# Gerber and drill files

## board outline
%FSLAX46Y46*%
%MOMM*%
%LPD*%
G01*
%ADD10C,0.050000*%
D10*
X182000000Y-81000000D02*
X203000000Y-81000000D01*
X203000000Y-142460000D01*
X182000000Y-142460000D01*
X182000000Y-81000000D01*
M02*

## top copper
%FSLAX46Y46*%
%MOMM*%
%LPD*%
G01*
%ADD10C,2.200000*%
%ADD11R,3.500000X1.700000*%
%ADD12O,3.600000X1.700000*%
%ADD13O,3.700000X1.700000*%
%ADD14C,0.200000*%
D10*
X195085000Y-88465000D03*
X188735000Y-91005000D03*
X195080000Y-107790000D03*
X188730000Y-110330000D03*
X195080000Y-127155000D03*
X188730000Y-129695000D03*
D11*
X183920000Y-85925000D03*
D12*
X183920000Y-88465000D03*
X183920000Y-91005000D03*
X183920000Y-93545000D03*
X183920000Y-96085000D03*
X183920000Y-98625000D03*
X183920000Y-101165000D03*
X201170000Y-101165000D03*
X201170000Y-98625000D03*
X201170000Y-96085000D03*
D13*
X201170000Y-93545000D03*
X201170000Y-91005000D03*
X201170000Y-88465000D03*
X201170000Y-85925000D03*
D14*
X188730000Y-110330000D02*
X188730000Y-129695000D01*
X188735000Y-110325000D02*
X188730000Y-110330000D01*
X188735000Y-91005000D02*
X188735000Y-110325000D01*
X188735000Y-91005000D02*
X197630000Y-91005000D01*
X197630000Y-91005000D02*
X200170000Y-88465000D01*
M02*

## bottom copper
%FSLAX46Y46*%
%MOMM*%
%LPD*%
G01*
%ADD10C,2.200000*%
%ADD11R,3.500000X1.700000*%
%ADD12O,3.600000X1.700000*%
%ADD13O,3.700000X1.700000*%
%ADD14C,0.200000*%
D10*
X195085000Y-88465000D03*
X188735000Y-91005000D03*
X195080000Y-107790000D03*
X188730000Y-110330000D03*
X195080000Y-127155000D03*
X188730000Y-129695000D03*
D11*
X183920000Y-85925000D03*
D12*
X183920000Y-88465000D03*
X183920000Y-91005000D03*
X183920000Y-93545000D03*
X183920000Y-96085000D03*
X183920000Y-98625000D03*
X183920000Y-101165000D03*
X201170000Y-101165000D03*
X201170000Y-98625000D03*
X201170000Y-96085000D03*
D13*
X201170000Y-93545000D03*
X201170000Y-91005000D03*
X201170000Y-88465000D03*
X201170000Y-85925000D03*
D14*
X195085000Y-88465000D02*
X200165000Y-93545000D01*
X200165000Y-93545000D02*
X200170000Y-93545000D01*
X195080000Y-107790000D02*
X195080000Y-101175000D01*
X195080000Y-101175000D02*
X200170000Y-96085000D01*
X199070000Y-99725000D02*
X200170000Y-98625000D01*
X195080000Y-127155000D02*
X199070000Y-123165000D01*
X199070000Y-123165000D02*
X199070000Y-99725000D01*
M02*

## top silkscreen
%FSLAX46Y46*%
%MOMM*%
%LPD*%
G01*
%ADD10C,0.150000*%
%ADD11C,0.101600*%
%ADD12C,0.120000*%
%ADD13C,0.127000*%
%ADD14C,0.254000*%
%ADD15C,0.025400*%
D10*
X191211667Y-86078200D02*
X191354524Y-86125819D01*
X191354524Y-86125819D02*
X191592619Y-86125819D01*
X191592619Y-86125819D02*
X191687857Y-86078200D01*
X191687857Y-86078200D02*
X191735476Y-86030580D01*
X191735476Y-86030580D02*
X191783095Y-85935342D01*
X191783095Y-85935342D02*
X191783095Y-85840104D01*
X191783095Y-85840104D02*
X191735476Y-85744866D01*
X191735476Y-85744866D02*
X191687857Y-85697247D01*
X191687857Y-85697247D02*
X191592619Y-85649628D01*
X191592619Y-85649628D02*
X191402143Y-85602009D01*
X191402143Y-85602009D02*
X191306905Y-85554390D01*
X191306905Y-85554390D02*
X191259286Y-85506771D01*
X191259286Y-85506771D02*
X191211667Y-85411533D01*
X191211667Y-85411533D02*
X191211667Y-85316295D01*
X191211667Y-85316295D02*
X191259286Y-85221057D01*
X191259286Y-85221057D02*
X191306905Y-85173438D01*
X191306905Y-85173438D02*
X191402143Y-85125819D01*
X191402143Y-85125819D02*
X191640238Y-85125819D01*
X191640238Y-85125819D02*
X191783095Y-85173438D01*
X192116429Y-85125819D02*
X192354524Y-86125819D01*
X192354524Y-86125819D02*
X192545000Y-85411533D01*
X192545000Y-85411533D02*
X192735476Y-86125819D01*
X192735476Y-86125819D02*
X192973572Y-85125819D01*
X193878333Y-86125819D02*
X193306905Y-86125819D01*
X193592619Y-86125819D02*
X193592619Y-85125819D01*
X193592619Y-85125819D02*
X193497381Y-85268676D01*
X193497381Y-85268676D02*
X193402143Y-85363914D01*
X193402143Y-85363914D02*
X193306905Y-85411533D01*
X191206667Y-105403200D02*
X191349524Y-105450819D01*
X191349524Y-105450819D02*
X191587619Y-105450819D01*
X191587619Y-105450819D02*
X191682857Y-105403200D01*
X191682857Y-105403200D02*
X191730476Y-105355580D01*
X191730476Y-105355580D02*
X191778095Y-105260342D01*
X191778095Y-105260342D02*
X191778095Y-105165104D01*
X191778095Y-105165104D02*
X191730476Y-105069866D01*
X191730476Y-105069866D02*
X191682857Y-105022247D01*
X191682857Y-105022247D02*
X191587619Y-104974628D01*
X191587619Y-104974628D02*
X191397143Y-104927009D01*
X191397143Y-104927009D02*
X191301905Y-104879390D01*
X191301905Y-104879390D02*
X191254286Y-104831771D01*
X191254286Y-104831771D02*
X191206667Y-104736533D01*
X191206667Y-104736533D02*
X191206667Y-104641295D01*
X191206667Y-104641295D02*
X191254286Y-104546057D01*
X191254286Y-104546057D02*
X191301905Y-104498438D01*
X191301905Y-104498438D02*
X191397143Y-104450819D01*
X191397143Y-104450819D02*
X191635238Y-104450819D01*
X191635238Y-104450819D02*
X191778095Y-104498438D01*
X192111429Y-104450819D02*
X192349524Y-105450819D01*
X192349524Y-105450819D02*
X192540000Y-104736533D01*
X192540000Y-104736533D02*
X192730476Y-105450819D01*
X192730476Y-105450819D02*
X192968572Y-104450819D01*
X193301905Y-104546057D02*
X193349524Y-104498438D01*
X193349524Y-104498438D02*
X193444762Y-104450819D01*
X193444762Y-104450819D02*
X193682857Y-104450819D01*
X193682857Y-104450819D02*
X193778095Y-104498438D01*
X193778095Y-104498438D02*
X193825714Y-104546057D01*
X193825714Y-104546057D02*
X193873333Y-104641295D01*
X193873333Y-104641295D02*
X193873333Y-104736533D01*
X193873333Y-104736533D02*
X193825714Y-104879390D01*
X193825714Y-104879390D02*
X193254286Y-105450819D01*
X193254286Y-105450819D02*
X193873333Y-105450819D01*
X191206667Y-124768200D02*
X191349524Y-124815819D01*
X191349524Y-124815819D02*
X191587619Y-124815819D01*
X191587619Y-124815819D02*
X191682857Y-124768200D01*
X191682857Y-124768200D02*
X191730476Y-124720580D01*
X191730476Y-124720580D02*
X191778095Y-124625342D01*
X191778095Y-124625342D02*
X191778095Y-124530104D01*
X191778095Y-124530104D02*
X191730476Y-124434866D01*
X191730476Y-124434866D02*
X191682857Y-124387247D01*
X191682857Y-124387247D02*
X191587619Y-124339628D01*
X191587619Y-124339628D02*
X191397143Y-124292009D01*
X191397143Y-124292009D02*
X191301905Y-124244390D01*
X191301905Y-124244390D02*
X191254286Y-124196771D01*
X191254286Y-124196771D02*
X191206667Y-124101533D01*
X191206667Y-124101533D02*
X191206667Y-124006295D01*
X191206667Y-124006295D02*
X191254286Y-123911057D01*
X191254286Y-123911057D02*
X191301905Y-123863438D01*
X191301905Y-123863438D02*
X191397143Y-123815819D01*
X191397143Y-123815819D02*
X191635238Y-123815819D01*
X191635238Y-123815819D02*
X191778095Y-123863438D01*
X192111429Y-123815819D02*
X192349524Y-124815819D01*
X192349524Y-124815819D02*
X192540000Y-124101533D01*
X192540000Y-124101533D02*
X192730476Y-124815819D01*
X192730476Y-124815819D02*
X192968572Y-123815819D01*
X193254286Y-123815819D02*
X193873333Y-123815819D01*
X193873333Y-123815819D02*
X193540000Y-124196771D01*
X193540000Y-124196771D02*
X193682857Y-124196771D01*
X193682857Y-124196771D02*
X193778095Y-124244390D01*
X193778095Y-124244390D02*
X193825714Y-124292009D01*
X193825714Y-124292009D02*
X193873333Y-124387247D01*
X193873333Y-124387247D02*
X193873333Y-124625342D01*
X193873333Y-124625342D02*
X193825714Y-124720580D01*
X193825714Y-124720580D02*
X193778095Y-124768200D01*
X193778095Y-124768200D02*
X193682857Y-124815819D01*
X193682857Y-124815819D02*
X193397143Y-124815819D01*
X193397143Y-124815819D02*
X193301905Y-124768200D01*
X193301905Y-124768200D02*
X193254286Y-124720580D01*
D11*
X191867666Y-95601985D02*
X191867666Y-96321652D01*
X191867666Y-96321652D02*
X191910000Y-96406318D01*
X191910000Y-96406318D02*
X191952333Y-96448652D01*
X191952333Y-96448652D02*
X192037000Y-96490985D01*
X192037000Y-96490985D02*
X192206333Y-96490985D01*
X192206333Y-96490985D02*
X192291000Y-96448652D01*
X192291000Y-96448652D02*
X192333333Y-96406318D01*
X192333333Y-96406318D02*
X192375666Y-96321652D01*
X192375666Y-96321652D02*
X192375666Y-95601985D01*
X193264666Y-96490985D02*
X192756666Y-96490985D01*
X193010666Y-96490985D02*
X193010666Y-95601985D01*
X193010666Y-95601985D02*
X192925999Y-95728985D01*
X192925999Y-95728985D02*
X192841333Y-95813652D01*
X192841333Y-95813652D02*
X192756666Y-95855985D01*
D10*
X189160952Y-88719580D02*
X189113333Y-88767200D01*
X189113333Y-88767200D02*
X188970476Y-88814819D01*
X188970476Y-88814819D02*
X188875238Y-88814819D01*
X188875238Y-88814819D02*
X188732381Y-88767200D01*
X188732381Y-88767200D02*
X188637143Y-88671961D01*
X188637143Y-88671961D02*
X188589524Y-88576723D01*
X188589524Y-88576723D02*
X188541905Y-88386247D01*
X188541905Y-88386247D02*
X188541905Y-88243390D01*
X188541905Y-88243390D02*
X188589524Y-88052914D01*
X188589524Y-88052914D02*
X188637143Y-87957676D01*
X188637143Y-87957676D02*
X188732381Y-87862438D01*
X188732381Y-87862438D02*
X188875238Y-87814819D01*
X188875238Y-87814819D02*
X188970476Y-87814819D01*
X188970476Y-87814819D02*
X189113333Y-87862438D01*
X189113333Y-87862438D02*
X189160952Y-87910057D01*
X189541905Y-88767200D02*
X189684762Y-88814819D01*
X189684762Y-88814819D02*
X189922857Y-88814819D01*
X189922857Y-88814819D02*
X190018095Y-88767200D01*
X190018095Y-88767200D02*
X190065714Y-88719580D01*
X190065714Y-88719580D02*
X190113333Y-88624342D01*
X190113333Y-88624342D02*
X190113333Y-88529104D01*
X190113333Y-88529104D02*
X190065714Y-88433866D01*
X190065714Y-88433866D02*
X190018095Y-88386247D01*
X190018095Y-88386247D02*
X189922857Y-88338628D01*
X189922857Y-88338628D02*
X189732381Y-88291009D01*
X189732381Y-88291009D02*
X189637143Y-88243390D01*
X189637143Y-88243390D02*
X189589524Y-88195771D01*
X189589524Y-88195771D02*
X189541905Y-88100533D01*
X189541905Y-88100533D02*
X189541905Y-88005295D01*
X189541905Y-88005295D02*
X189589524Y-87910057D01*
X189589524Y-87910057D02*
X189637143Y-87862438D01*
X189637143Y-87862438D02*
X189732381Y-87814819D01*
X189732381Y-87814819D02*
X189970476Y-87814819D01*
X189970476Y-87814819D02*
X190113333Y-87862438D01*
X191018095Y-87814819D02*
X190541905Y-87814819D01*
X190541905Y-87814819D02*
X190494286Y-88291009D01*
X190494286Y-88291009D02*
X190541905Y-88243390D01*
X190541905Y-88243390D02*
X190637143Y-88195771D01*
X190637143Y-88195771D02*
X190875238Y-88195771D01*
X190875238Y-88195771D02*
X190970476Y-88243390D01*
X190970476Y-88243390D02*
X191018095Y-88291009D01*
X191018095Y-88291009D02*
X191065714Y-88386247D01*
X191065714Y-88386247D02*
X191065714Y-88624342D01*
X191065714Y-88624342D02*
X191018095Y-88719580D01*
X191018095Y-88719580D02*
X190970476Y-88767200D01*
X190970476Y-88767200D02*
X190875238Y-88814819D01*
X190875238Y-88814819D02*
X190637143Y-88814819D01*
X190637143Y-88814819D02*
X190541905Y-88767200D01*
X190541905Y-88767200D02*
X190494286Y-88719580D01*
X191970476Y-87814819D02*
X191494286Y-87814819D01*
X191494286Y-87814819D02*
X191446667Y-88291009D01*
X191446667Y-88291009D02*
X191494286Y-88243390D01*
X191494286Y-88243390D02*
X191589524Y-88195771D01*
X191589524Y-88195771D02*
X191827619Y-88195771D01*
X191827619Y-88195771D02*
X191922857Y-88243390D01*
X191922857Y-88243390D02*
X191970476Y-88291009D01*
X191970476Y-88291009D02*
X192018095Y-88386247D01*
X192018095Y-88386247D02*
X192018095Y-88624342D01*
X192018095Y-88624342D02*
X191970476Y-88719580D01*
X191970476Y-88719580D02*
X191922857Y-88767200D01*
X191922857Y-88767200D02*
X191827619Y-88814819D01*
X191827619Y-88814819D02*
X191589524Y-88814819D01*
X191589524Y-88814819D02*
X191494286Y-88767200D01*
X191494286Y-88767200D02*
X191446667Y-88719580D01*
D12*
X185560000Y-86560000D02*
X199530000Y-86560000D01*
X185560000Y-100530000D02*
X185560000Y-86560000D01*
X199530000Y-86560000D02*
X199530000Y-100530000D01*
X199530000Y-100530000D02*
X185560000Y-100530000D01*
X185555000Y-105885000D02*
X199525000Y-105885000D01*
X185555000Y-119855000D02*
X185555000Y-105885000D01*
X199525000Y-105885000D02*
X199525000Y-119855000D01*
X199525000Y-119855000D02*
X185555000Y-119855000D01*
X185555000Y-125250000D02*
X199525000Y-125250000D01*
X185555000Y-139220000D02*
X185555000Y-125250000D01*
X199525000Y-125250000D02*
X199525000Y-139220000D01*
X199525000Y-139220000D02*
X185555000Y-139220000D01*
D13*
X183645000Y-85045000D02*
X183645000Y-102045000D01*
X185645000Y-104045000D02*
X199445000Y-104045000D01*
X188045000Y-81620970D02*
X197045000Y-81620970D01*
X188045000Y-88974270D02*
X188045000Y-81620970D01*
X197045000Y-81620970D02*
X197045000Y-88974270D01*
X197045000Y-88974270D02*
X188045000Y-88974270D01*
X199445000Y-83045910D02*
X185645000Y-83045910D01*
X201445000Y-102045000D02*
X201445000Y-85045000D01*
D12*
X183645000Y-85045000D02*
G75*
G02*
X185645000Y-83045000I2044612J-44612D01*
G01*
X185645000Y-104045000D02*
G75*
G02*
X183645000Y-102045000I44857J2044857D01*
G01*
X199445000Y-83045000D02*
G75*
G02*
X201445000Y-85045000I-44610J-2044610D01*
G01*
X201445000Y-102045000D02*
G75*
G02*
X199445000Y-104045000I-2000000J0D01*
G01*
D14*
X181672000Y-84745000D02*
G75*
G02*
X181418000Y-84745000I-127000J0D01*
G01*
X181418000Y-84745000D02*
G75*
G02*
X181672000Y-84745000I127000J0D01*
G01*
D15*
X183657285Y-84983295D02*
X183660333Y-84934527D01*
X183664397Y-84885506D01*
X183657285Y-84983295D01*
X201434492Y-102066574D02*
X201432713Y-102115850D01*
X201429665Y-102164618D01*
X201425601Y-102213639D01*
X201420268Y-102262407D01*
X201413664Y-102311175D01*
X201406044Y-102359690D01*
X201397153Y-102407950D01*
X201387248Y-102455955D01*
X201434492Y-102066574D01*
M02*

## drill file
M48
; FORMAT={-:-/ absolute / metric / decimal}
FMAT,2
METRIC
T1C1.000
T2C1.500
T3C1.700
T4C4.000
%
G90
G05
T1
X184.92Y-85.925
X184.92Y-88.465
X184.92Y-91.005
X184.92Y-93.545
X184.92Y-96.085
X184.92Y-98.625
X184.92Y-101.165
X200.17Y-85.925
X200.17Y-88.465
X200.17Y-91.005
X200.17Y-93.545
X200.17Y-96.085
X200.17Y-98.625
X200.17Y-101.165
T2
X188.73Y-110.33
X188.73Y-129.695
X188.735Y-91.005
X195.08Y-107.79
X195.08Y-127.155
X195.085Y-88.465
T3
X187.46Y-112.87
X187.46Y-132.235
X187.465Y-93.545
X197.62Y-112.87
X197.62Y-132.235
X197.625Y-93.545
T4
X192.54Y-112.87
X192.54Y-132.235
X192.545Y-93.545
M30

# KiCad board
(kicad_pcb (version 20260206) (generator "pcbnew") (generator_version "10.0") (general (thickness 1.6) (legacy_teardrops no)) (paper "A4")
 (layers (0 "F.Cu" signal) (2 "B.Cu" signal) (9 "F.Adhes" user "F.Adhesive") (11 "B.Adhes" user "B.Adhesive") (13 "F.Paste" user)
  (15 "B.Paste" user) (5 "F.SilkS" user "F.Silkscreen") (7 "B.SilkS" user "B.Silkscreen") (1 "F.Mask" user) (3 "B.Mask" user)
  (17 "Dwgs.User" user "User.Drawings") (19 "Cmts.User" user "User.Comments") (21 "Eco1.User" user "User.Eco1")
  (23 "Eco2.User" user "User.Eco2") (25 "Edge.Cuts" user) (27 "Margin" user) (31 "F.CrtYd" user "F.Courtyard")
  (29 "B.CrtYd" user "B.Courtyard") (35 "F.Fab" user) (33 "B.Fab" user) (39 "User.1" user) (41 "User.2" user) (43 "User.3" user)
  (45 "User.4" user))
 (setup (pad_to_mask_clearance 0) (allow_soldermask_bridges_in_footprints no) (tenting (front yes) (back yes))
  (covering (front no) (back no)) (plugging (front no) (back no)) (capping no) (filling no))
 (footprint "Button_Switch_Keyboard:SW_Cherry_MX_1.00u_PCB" (layer "F.Cu") (at 195.085 88.465)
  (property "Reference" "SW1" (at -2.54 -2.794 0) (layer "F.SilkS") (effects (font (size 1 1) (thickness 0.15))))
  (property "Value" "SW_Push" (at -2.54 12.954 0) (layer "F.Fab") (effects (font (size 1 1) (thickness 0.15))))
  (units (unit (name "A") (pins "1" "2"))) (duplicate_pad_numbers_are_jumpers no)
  (fp_line (start -9.525 -1.905) (end 4.445 -1.905) (stroke (width 0.12) (type solid)) (layer "F.SilkS"))
  (fp_line (start -9.525 12.065) (end -9.525 -1.905) (stroke (width 0.12) (type solid)) (layer "F.SilkS"))
  (fp_line (start 4.445 -1.905) (end 4.445 12.065) (stroke (width 0.12) (type solid)) (layer "F.SilkS"))
  (fp_line (start 4.445 12.065) (end -9.525 12.065) (stroke (width 0.12) (type solid)) (layer "F.SilkS"))
  (pad "" np_thru_hole circle (at -7.62 5.08) (size 1.7 1.7) (drill 1.7) (layers "*.Cu" "*.Mask"))
  (pad "" np_thru_hole circle (at -2.54 5.08) (size 4 4) (drill 4) (layers "*.Cu" "*.Mask"))
  (pad "" np_thru_hole circle (at 2.54 5.08) (size 1.7 1.7) (drill 1.7) (layers "*.Cu" "*.Mask"))
  (pad "1" thru_hole circle (at 0 0) (size 2.2 2.2) (drill 1.5) (layers "*.Cu" "*.Mask") (remove_unused_layers no)
   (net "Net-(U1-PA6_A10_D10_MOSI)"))
  (pad "2" thru_hole circle (at -6.35 2.54) (size 2.2 2.2) (drill 1.5) (layers "*.Cu" "*.Mask") (remove_unused_layers no) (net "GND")))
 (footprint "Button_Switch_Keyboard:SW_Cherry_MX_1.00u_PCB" (layer "F.Cu") (at 195.08 107.79)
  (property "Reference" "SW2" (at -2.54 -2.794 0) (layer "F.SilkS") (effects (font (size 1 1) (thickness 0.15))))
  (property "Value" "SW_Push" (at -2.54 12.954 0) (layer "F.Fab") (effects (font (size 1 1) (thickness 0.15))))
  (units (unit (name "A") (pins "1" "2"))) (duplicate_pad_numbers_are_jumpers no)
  (fp_line (start -9.525 -1.905) (end 4.445 -1.905) (stroke (width 0.12) (type solid)) (layer "F.SilkS"))
  (fp_line (start -9.525 12.065) (end -9.525 -1.905) (stroke (width 0.12) (type solid)) (layer "F.SilkS"))
  (fp_line (start 4.445 -1.905) (end 4.445 12.065) (stroke (width 0.12) (type solid)) (layer "F.SilkS"))
  (fp_line (start 4.445 12.065) (end -9.525 12.065) (stroke (width 0.12) (type solid)) (layer "F.SilkS"))
  (pad "" np_thru_hole circle (at -7.62 5.08) (size 1.7 1.7) (drill 1.7) (layers "*.Cu" "*.Mask"))
  (pad "" np_thru_hole circle (at -2.54 5.08) (size 4 4) (drill 4) (layers "*.Cu" "*.Mask"))
  (pad "" np_thru_hole circle (at 2.54 5.08) (size 1.7 1.7) (drill 1.7) (layers "*.Cu" "*.Mask"))
  (pad "1" thru_hole circle (at 0 0) (size 2.2 2.2) (drill 1.5) (layers "*.Cu" "*.Mask") (remove_unused_layers no)
   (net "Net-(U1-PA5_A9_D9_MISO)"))
  (pad "2" thru_hole circle (at -6.35 2.54) (size 2.2 2.2) (drill 1.5) (layers "*.Cu" "*.Mask") (remove_unused_layers no) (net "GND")))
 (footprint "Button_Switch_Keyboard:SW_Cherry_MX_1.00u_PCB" (layer "F.Cu") (at 195.08 127.155)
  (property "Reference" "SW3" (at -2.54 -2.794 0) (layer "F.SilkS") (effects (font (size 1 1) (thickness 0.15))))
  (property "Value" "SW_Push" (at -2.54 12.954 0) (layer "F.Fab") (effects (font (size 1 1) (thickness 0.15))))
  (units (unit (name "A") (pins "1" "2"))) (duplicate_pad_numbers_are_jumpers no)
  (fp_line (start -9.525 -1.905) (end 4.445 -1.905) (stroke (width 0.12) (type solid)) (layer "F.SilkS"))
  (fp_line (start -9.525 12.065) (end -9.525 -1.905) (stroke (width 0.12) (type solid)) (layer "F.SilkS"))
  (fp_line (start 4.445 -1.905) (end 4.445 12.065) (stroke (width 0.12) (type solid)) (layer "F.SilkS"))
  (fp_line (start 4.445 12.065) (end -9.525 12.065) (stroke (width 0.12) (type solid)) (layer "F.SilkS"))
  (pad "" np_thru_hole circle (at -7.62 5.08) (size 1.7 1.7) (drill 1.7) (layers "*.Cu" "*.Mask"))
  (pad "" np_thru_hole circle (at -2.54 5.08) (size 4 4) (drill 4) (layers "*.Cu" "*.Mask"))
  (pad "" np_thru_hole circle (at 2.54 5.08) (size 1.7 1.7) (drill 1.7) (layers "*.Cu" "*.Mask"))
  (pad "1" thru_hole circle (at 0 0) (size 2.2 2.2) (drill 1.5) (layers "*.Cu" "*.Mask") (remove_unused_layers no)
   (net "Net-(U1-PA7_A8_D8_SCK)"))
  (pad "2" thru_hole circle (at -6.35 2.54) (size 2.2 2.2) (drill 1.5) (layers "*.Cu" "*.Mask") (remove_unused_layers no) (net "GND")))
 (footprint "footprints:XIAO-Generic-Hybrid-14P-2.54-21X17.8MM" (layer "F.Cu") (at 192.545 93.545)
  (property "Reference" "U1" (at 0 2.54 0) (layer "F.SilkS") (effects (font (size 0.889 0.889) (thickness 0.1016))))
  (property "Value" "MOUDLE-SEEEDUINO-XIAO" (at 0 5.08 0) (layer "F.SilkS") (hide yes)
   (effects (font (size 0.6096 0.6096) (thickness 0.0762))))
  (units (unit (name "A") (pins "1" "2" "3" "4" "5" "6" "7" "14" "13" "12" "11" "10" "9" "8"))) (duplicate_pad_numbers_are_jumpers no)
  (fp_line (start -8.9 -8.5) (end -8.9 8.5) (stroke (width 0.127) (type solid)) (layer "F.SilkS"))
  (fp_line (start -6.9 10.5) (end 6.9 10.5) (stroke (width 0.127) (type solid)) (layer "F.SilkS"))
  (fp_line (start -4.5 -11.92403) (end 4.5 -11.92403) (stroke (width 0.127) (type solid)) (layer "F.SilkS"))
  (fp_line (start -4.5 -4.57073) (end -4.5 -11.92403) (stroke (width 0.127) (type solid)) (layer "F.SilkS"))
  (fp_line (start 4.5 -11.92403) (end 4.5 -4.57073) (stroke (width 0.127) (type solid)) (layer "F.SilkS"))
  (fp_line (start 4.5 -4.57073) (end -4.5 -4.57073) (stroke (width 0.127) (type solid)) (layer "F.SilkS"))
  (fp_line (start 6.9 -10.49909) (end -6.9 -10.49909) (stroke (width 0.127) (type solid)) (layer "F.SilkS"))
  (fp_line (start 8.9 8.5) (end 8.9 -8.5) (stroke (width 0.127) (type solid)) (layer "F.SilkS"))
  (fp_arc (start -8.9 -8.5) (mid -8.301491 -9.901491) (end -6.9 -10.5) (stroke (width 0.12) (type solid)) (layer "F.SilkS"))
  (fp_arc (start -6.9 10.5) (mid -8.301423 9.901423) (end -8.9 8.5) (stroke (width 0.12) (type solid)) (layer "F.SilkS"))
  (fp_arc (start 6.9 -10.5) (mid 8.301491 -9.901491) (end 8.9 -8.5) (stroke (width 0.12) (type solid)) (layer "F.SilkS"))
  (fp_arc (start 8.9 8.5) (mid 8.314214 9.914214) (end 6.9 10.5) (stroke (width 0.12) (type solid)) (layer "F.SilkS"))
  (fp_circle (center -11 -8.8) (end -11 -9.054) (stroke (width 0) (type solid)) (fill yes) (layer "F.SilkS"))
  (fp_poly
   (pts (xy -8.887715 -8.561705) (xy -8.884667 -8.610473) (xy -8.880603 -8.659494)) (stroke (width 0.0254) (type solid)) (fill no)
   (layer "F.SilkS"))
  (fp_poly
   (pts (xy 8.889492 8.521574) (xy 8.887713 8.57085) (xy 8.884665 8.619618) (xy 8.880601 8.668639) (xy 8.875268 8.717407)
    (xy 8.868664 8.766175) (xy 8.861044 8.81469) (xy 8.852153 8.86295) (xy 8.842248 8.910955))
   (stroke (width 0.0254) (type solid)) (fill no) (layer "F.SilkS"))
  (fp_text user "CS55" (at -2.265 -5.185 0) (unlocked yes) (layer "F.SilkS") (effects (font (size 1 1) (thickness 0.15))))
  (pad "1" thru_hole rect (at -7.625 -7.62) (size 3.5 1.7) (drill 1 (offset -1 0)) (layers "*.Cu" "*.Mask") (remove_unused_layers no)
   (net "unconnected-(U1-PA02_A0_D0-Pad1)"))
  (pad "2" thru_hole oval (at -7.625 -5.08) (size 3.6 1.7) (drill 1 (offset -1 0)) (layers "*.Cu" "*.Mask") (remove_unused_layers no)
   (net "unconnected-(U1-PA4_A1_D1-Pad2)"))
  (pad "3" thru_hole oval (at -7.625 -2.54) (size 3.6 1.7) (drill 1 (offset -1 0)) (layers "*.Cu" "*.Mask") (remove_unused_layers no)
   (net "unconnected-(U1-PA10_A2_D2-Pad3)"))
  (pad "4" thru_hole oval (at -7.625 0) (size 3.6 1.7) (drill 1 (offset -1 0)) (layers "*.Cu" "*.Mask") (remove_unused_layers no)
   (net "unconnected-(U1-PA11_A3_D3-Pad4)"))
  (pad "5" thru_hole oval (at -7.625 2.54) (size 3.6 1.7) (drill 1 (offset -1 0)) (layers "*.Cu" "*.Mask") (remove_unused_layers no)
   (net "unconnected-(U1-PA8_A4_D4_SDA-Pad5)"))
  (pad "6" thru_hole oval (at -7.625 5.08 180) (size 3.6 1.7) (drill 1 (offset 1 0)) (layers "*.Cu" "*.Mask") (remove_unused_layers no)
   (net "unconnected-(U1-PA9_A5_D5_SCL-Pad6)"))
  (pad "7" thru_hole oval (at -7.625 7.62) (size 3.6 1.7) (drill 1 (offset -1 0)) (layers "*.Cu" "*.Mask") (remove_unused_layers no)
   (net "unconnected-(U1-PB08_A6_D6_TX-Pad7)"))
  (pad "8" thru_hole oval (at 7.625 7.62) (size 3.6 1.7) (drill 1 (offset 1 0)) (layers "*.Cu" "*.Mask") (remove_unused_layers no)
   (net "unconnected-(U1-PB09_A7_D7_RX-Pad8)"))
  (pad "9" thru_hole oval (at 7.625 5.08) (size 3.6 1.7) (drill 1 (offset 1 0)) (layers "*.Cu" "*.Mask") (remove_unused_layers no)
   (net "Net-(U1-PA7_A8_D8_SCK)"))
  (pad "10" thru_hole oval (at 7.625 2.54) (size 3.6 1.7) (drill 1 (offset 1 0)) (layers "*.Cu" "*.Mask") (remove_unused_layers no)
   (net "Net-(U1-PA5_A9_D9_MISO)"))
  (pad "11" thru_hole oval (at 7.625 0) (size 3.7 1.7) (drill 1 (offset 1 0)) (layers "*.Cu" "*.Mask") (remove_unused_layers no)
   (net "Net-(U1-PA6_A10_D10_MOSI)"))
  (pad "12" thru_hole oval (at 7.625 -2.54) (size 3.7 1.7) (drill 1 (offset 1 0)) (layers "*.Cu" "*.Mask") (remove_unused_layers no)
   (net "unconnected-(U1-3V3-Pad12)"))
  (pad "13" thru_hole oval (at 7.625 -5.08) (size 3.7 1.7) (drill 1 (offset 1 0)) (layers "*.Cu" "*.Mask") (remove_unused_layers no)
   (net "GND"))
  (pad "14" thru_hole oval (at 7.625 -7.62) (size 3.7 1.7) (drill 1 (offset 1 0)) (layers "*.Cu" "*.Mask") (remove_unused_layers no)
   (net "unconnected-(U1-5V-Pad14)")))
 (gr_rect (start 182 81) (end 203 142.46) (stroke (width 0.05) (type default)) (fill no) (layer "Edge.Cuts"))
 (segment (start 195.085 88.465) (end 200.165 93.545) (width 0.2) (layer "B.Cu") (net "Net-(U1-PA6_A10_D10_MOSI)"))
 (segment (start 200.165 93.545) (end 200.17 93.545) (width 0.2) (layer "B.Cu") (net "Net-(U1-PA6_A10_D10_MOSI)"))
 (segment (start 188.73 110.33) (end 188.73 129.695) (width 0.2) (layer "F.Cu") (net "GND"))
 (segment (start 188.735 110.325) (end 188.73 110.33) (width 0.2) (layer "F.Cu") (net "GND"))
 (segment (start 188.735 91.005) (end 188.735 110.325) (width 0.2) (layer "F.Cu") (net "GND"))
 (segment (start 188.735 91.005) (end 197.63 91.005) (width 0.2) (layer "F.Cu") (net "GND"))
 (segment (start 197.63 91.005) (end 200.17 88.465) (width 0.2) (layer "F.Cu") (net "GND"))
 (segment (start 195.08 107.79) (end 195.08 101.175) (width 0.2) (layer "B.Cu") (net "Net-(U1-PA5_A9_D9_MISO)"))
 (segment (start 195.08 101.175) (end 200.17 96.085) (width 0.2) (layer "B.Cu") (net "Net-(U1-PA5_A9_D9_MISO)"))
 (segment (start 199.07 99.725) (end 200.17 98.625) (width 0.2) (layer "B.Cu") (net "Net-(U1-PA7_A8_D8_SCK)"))
 (segment (start 195.08 127.155) (end 199.07 123.165) (width 0.2) (layer "B.Cu") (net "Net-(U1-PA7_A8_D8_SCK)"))
 (segment (start 199.07 123.165) (end 199.07 99.725) (width 0.2) (layer "B.Cu") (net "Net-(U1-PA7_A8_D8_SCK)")))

